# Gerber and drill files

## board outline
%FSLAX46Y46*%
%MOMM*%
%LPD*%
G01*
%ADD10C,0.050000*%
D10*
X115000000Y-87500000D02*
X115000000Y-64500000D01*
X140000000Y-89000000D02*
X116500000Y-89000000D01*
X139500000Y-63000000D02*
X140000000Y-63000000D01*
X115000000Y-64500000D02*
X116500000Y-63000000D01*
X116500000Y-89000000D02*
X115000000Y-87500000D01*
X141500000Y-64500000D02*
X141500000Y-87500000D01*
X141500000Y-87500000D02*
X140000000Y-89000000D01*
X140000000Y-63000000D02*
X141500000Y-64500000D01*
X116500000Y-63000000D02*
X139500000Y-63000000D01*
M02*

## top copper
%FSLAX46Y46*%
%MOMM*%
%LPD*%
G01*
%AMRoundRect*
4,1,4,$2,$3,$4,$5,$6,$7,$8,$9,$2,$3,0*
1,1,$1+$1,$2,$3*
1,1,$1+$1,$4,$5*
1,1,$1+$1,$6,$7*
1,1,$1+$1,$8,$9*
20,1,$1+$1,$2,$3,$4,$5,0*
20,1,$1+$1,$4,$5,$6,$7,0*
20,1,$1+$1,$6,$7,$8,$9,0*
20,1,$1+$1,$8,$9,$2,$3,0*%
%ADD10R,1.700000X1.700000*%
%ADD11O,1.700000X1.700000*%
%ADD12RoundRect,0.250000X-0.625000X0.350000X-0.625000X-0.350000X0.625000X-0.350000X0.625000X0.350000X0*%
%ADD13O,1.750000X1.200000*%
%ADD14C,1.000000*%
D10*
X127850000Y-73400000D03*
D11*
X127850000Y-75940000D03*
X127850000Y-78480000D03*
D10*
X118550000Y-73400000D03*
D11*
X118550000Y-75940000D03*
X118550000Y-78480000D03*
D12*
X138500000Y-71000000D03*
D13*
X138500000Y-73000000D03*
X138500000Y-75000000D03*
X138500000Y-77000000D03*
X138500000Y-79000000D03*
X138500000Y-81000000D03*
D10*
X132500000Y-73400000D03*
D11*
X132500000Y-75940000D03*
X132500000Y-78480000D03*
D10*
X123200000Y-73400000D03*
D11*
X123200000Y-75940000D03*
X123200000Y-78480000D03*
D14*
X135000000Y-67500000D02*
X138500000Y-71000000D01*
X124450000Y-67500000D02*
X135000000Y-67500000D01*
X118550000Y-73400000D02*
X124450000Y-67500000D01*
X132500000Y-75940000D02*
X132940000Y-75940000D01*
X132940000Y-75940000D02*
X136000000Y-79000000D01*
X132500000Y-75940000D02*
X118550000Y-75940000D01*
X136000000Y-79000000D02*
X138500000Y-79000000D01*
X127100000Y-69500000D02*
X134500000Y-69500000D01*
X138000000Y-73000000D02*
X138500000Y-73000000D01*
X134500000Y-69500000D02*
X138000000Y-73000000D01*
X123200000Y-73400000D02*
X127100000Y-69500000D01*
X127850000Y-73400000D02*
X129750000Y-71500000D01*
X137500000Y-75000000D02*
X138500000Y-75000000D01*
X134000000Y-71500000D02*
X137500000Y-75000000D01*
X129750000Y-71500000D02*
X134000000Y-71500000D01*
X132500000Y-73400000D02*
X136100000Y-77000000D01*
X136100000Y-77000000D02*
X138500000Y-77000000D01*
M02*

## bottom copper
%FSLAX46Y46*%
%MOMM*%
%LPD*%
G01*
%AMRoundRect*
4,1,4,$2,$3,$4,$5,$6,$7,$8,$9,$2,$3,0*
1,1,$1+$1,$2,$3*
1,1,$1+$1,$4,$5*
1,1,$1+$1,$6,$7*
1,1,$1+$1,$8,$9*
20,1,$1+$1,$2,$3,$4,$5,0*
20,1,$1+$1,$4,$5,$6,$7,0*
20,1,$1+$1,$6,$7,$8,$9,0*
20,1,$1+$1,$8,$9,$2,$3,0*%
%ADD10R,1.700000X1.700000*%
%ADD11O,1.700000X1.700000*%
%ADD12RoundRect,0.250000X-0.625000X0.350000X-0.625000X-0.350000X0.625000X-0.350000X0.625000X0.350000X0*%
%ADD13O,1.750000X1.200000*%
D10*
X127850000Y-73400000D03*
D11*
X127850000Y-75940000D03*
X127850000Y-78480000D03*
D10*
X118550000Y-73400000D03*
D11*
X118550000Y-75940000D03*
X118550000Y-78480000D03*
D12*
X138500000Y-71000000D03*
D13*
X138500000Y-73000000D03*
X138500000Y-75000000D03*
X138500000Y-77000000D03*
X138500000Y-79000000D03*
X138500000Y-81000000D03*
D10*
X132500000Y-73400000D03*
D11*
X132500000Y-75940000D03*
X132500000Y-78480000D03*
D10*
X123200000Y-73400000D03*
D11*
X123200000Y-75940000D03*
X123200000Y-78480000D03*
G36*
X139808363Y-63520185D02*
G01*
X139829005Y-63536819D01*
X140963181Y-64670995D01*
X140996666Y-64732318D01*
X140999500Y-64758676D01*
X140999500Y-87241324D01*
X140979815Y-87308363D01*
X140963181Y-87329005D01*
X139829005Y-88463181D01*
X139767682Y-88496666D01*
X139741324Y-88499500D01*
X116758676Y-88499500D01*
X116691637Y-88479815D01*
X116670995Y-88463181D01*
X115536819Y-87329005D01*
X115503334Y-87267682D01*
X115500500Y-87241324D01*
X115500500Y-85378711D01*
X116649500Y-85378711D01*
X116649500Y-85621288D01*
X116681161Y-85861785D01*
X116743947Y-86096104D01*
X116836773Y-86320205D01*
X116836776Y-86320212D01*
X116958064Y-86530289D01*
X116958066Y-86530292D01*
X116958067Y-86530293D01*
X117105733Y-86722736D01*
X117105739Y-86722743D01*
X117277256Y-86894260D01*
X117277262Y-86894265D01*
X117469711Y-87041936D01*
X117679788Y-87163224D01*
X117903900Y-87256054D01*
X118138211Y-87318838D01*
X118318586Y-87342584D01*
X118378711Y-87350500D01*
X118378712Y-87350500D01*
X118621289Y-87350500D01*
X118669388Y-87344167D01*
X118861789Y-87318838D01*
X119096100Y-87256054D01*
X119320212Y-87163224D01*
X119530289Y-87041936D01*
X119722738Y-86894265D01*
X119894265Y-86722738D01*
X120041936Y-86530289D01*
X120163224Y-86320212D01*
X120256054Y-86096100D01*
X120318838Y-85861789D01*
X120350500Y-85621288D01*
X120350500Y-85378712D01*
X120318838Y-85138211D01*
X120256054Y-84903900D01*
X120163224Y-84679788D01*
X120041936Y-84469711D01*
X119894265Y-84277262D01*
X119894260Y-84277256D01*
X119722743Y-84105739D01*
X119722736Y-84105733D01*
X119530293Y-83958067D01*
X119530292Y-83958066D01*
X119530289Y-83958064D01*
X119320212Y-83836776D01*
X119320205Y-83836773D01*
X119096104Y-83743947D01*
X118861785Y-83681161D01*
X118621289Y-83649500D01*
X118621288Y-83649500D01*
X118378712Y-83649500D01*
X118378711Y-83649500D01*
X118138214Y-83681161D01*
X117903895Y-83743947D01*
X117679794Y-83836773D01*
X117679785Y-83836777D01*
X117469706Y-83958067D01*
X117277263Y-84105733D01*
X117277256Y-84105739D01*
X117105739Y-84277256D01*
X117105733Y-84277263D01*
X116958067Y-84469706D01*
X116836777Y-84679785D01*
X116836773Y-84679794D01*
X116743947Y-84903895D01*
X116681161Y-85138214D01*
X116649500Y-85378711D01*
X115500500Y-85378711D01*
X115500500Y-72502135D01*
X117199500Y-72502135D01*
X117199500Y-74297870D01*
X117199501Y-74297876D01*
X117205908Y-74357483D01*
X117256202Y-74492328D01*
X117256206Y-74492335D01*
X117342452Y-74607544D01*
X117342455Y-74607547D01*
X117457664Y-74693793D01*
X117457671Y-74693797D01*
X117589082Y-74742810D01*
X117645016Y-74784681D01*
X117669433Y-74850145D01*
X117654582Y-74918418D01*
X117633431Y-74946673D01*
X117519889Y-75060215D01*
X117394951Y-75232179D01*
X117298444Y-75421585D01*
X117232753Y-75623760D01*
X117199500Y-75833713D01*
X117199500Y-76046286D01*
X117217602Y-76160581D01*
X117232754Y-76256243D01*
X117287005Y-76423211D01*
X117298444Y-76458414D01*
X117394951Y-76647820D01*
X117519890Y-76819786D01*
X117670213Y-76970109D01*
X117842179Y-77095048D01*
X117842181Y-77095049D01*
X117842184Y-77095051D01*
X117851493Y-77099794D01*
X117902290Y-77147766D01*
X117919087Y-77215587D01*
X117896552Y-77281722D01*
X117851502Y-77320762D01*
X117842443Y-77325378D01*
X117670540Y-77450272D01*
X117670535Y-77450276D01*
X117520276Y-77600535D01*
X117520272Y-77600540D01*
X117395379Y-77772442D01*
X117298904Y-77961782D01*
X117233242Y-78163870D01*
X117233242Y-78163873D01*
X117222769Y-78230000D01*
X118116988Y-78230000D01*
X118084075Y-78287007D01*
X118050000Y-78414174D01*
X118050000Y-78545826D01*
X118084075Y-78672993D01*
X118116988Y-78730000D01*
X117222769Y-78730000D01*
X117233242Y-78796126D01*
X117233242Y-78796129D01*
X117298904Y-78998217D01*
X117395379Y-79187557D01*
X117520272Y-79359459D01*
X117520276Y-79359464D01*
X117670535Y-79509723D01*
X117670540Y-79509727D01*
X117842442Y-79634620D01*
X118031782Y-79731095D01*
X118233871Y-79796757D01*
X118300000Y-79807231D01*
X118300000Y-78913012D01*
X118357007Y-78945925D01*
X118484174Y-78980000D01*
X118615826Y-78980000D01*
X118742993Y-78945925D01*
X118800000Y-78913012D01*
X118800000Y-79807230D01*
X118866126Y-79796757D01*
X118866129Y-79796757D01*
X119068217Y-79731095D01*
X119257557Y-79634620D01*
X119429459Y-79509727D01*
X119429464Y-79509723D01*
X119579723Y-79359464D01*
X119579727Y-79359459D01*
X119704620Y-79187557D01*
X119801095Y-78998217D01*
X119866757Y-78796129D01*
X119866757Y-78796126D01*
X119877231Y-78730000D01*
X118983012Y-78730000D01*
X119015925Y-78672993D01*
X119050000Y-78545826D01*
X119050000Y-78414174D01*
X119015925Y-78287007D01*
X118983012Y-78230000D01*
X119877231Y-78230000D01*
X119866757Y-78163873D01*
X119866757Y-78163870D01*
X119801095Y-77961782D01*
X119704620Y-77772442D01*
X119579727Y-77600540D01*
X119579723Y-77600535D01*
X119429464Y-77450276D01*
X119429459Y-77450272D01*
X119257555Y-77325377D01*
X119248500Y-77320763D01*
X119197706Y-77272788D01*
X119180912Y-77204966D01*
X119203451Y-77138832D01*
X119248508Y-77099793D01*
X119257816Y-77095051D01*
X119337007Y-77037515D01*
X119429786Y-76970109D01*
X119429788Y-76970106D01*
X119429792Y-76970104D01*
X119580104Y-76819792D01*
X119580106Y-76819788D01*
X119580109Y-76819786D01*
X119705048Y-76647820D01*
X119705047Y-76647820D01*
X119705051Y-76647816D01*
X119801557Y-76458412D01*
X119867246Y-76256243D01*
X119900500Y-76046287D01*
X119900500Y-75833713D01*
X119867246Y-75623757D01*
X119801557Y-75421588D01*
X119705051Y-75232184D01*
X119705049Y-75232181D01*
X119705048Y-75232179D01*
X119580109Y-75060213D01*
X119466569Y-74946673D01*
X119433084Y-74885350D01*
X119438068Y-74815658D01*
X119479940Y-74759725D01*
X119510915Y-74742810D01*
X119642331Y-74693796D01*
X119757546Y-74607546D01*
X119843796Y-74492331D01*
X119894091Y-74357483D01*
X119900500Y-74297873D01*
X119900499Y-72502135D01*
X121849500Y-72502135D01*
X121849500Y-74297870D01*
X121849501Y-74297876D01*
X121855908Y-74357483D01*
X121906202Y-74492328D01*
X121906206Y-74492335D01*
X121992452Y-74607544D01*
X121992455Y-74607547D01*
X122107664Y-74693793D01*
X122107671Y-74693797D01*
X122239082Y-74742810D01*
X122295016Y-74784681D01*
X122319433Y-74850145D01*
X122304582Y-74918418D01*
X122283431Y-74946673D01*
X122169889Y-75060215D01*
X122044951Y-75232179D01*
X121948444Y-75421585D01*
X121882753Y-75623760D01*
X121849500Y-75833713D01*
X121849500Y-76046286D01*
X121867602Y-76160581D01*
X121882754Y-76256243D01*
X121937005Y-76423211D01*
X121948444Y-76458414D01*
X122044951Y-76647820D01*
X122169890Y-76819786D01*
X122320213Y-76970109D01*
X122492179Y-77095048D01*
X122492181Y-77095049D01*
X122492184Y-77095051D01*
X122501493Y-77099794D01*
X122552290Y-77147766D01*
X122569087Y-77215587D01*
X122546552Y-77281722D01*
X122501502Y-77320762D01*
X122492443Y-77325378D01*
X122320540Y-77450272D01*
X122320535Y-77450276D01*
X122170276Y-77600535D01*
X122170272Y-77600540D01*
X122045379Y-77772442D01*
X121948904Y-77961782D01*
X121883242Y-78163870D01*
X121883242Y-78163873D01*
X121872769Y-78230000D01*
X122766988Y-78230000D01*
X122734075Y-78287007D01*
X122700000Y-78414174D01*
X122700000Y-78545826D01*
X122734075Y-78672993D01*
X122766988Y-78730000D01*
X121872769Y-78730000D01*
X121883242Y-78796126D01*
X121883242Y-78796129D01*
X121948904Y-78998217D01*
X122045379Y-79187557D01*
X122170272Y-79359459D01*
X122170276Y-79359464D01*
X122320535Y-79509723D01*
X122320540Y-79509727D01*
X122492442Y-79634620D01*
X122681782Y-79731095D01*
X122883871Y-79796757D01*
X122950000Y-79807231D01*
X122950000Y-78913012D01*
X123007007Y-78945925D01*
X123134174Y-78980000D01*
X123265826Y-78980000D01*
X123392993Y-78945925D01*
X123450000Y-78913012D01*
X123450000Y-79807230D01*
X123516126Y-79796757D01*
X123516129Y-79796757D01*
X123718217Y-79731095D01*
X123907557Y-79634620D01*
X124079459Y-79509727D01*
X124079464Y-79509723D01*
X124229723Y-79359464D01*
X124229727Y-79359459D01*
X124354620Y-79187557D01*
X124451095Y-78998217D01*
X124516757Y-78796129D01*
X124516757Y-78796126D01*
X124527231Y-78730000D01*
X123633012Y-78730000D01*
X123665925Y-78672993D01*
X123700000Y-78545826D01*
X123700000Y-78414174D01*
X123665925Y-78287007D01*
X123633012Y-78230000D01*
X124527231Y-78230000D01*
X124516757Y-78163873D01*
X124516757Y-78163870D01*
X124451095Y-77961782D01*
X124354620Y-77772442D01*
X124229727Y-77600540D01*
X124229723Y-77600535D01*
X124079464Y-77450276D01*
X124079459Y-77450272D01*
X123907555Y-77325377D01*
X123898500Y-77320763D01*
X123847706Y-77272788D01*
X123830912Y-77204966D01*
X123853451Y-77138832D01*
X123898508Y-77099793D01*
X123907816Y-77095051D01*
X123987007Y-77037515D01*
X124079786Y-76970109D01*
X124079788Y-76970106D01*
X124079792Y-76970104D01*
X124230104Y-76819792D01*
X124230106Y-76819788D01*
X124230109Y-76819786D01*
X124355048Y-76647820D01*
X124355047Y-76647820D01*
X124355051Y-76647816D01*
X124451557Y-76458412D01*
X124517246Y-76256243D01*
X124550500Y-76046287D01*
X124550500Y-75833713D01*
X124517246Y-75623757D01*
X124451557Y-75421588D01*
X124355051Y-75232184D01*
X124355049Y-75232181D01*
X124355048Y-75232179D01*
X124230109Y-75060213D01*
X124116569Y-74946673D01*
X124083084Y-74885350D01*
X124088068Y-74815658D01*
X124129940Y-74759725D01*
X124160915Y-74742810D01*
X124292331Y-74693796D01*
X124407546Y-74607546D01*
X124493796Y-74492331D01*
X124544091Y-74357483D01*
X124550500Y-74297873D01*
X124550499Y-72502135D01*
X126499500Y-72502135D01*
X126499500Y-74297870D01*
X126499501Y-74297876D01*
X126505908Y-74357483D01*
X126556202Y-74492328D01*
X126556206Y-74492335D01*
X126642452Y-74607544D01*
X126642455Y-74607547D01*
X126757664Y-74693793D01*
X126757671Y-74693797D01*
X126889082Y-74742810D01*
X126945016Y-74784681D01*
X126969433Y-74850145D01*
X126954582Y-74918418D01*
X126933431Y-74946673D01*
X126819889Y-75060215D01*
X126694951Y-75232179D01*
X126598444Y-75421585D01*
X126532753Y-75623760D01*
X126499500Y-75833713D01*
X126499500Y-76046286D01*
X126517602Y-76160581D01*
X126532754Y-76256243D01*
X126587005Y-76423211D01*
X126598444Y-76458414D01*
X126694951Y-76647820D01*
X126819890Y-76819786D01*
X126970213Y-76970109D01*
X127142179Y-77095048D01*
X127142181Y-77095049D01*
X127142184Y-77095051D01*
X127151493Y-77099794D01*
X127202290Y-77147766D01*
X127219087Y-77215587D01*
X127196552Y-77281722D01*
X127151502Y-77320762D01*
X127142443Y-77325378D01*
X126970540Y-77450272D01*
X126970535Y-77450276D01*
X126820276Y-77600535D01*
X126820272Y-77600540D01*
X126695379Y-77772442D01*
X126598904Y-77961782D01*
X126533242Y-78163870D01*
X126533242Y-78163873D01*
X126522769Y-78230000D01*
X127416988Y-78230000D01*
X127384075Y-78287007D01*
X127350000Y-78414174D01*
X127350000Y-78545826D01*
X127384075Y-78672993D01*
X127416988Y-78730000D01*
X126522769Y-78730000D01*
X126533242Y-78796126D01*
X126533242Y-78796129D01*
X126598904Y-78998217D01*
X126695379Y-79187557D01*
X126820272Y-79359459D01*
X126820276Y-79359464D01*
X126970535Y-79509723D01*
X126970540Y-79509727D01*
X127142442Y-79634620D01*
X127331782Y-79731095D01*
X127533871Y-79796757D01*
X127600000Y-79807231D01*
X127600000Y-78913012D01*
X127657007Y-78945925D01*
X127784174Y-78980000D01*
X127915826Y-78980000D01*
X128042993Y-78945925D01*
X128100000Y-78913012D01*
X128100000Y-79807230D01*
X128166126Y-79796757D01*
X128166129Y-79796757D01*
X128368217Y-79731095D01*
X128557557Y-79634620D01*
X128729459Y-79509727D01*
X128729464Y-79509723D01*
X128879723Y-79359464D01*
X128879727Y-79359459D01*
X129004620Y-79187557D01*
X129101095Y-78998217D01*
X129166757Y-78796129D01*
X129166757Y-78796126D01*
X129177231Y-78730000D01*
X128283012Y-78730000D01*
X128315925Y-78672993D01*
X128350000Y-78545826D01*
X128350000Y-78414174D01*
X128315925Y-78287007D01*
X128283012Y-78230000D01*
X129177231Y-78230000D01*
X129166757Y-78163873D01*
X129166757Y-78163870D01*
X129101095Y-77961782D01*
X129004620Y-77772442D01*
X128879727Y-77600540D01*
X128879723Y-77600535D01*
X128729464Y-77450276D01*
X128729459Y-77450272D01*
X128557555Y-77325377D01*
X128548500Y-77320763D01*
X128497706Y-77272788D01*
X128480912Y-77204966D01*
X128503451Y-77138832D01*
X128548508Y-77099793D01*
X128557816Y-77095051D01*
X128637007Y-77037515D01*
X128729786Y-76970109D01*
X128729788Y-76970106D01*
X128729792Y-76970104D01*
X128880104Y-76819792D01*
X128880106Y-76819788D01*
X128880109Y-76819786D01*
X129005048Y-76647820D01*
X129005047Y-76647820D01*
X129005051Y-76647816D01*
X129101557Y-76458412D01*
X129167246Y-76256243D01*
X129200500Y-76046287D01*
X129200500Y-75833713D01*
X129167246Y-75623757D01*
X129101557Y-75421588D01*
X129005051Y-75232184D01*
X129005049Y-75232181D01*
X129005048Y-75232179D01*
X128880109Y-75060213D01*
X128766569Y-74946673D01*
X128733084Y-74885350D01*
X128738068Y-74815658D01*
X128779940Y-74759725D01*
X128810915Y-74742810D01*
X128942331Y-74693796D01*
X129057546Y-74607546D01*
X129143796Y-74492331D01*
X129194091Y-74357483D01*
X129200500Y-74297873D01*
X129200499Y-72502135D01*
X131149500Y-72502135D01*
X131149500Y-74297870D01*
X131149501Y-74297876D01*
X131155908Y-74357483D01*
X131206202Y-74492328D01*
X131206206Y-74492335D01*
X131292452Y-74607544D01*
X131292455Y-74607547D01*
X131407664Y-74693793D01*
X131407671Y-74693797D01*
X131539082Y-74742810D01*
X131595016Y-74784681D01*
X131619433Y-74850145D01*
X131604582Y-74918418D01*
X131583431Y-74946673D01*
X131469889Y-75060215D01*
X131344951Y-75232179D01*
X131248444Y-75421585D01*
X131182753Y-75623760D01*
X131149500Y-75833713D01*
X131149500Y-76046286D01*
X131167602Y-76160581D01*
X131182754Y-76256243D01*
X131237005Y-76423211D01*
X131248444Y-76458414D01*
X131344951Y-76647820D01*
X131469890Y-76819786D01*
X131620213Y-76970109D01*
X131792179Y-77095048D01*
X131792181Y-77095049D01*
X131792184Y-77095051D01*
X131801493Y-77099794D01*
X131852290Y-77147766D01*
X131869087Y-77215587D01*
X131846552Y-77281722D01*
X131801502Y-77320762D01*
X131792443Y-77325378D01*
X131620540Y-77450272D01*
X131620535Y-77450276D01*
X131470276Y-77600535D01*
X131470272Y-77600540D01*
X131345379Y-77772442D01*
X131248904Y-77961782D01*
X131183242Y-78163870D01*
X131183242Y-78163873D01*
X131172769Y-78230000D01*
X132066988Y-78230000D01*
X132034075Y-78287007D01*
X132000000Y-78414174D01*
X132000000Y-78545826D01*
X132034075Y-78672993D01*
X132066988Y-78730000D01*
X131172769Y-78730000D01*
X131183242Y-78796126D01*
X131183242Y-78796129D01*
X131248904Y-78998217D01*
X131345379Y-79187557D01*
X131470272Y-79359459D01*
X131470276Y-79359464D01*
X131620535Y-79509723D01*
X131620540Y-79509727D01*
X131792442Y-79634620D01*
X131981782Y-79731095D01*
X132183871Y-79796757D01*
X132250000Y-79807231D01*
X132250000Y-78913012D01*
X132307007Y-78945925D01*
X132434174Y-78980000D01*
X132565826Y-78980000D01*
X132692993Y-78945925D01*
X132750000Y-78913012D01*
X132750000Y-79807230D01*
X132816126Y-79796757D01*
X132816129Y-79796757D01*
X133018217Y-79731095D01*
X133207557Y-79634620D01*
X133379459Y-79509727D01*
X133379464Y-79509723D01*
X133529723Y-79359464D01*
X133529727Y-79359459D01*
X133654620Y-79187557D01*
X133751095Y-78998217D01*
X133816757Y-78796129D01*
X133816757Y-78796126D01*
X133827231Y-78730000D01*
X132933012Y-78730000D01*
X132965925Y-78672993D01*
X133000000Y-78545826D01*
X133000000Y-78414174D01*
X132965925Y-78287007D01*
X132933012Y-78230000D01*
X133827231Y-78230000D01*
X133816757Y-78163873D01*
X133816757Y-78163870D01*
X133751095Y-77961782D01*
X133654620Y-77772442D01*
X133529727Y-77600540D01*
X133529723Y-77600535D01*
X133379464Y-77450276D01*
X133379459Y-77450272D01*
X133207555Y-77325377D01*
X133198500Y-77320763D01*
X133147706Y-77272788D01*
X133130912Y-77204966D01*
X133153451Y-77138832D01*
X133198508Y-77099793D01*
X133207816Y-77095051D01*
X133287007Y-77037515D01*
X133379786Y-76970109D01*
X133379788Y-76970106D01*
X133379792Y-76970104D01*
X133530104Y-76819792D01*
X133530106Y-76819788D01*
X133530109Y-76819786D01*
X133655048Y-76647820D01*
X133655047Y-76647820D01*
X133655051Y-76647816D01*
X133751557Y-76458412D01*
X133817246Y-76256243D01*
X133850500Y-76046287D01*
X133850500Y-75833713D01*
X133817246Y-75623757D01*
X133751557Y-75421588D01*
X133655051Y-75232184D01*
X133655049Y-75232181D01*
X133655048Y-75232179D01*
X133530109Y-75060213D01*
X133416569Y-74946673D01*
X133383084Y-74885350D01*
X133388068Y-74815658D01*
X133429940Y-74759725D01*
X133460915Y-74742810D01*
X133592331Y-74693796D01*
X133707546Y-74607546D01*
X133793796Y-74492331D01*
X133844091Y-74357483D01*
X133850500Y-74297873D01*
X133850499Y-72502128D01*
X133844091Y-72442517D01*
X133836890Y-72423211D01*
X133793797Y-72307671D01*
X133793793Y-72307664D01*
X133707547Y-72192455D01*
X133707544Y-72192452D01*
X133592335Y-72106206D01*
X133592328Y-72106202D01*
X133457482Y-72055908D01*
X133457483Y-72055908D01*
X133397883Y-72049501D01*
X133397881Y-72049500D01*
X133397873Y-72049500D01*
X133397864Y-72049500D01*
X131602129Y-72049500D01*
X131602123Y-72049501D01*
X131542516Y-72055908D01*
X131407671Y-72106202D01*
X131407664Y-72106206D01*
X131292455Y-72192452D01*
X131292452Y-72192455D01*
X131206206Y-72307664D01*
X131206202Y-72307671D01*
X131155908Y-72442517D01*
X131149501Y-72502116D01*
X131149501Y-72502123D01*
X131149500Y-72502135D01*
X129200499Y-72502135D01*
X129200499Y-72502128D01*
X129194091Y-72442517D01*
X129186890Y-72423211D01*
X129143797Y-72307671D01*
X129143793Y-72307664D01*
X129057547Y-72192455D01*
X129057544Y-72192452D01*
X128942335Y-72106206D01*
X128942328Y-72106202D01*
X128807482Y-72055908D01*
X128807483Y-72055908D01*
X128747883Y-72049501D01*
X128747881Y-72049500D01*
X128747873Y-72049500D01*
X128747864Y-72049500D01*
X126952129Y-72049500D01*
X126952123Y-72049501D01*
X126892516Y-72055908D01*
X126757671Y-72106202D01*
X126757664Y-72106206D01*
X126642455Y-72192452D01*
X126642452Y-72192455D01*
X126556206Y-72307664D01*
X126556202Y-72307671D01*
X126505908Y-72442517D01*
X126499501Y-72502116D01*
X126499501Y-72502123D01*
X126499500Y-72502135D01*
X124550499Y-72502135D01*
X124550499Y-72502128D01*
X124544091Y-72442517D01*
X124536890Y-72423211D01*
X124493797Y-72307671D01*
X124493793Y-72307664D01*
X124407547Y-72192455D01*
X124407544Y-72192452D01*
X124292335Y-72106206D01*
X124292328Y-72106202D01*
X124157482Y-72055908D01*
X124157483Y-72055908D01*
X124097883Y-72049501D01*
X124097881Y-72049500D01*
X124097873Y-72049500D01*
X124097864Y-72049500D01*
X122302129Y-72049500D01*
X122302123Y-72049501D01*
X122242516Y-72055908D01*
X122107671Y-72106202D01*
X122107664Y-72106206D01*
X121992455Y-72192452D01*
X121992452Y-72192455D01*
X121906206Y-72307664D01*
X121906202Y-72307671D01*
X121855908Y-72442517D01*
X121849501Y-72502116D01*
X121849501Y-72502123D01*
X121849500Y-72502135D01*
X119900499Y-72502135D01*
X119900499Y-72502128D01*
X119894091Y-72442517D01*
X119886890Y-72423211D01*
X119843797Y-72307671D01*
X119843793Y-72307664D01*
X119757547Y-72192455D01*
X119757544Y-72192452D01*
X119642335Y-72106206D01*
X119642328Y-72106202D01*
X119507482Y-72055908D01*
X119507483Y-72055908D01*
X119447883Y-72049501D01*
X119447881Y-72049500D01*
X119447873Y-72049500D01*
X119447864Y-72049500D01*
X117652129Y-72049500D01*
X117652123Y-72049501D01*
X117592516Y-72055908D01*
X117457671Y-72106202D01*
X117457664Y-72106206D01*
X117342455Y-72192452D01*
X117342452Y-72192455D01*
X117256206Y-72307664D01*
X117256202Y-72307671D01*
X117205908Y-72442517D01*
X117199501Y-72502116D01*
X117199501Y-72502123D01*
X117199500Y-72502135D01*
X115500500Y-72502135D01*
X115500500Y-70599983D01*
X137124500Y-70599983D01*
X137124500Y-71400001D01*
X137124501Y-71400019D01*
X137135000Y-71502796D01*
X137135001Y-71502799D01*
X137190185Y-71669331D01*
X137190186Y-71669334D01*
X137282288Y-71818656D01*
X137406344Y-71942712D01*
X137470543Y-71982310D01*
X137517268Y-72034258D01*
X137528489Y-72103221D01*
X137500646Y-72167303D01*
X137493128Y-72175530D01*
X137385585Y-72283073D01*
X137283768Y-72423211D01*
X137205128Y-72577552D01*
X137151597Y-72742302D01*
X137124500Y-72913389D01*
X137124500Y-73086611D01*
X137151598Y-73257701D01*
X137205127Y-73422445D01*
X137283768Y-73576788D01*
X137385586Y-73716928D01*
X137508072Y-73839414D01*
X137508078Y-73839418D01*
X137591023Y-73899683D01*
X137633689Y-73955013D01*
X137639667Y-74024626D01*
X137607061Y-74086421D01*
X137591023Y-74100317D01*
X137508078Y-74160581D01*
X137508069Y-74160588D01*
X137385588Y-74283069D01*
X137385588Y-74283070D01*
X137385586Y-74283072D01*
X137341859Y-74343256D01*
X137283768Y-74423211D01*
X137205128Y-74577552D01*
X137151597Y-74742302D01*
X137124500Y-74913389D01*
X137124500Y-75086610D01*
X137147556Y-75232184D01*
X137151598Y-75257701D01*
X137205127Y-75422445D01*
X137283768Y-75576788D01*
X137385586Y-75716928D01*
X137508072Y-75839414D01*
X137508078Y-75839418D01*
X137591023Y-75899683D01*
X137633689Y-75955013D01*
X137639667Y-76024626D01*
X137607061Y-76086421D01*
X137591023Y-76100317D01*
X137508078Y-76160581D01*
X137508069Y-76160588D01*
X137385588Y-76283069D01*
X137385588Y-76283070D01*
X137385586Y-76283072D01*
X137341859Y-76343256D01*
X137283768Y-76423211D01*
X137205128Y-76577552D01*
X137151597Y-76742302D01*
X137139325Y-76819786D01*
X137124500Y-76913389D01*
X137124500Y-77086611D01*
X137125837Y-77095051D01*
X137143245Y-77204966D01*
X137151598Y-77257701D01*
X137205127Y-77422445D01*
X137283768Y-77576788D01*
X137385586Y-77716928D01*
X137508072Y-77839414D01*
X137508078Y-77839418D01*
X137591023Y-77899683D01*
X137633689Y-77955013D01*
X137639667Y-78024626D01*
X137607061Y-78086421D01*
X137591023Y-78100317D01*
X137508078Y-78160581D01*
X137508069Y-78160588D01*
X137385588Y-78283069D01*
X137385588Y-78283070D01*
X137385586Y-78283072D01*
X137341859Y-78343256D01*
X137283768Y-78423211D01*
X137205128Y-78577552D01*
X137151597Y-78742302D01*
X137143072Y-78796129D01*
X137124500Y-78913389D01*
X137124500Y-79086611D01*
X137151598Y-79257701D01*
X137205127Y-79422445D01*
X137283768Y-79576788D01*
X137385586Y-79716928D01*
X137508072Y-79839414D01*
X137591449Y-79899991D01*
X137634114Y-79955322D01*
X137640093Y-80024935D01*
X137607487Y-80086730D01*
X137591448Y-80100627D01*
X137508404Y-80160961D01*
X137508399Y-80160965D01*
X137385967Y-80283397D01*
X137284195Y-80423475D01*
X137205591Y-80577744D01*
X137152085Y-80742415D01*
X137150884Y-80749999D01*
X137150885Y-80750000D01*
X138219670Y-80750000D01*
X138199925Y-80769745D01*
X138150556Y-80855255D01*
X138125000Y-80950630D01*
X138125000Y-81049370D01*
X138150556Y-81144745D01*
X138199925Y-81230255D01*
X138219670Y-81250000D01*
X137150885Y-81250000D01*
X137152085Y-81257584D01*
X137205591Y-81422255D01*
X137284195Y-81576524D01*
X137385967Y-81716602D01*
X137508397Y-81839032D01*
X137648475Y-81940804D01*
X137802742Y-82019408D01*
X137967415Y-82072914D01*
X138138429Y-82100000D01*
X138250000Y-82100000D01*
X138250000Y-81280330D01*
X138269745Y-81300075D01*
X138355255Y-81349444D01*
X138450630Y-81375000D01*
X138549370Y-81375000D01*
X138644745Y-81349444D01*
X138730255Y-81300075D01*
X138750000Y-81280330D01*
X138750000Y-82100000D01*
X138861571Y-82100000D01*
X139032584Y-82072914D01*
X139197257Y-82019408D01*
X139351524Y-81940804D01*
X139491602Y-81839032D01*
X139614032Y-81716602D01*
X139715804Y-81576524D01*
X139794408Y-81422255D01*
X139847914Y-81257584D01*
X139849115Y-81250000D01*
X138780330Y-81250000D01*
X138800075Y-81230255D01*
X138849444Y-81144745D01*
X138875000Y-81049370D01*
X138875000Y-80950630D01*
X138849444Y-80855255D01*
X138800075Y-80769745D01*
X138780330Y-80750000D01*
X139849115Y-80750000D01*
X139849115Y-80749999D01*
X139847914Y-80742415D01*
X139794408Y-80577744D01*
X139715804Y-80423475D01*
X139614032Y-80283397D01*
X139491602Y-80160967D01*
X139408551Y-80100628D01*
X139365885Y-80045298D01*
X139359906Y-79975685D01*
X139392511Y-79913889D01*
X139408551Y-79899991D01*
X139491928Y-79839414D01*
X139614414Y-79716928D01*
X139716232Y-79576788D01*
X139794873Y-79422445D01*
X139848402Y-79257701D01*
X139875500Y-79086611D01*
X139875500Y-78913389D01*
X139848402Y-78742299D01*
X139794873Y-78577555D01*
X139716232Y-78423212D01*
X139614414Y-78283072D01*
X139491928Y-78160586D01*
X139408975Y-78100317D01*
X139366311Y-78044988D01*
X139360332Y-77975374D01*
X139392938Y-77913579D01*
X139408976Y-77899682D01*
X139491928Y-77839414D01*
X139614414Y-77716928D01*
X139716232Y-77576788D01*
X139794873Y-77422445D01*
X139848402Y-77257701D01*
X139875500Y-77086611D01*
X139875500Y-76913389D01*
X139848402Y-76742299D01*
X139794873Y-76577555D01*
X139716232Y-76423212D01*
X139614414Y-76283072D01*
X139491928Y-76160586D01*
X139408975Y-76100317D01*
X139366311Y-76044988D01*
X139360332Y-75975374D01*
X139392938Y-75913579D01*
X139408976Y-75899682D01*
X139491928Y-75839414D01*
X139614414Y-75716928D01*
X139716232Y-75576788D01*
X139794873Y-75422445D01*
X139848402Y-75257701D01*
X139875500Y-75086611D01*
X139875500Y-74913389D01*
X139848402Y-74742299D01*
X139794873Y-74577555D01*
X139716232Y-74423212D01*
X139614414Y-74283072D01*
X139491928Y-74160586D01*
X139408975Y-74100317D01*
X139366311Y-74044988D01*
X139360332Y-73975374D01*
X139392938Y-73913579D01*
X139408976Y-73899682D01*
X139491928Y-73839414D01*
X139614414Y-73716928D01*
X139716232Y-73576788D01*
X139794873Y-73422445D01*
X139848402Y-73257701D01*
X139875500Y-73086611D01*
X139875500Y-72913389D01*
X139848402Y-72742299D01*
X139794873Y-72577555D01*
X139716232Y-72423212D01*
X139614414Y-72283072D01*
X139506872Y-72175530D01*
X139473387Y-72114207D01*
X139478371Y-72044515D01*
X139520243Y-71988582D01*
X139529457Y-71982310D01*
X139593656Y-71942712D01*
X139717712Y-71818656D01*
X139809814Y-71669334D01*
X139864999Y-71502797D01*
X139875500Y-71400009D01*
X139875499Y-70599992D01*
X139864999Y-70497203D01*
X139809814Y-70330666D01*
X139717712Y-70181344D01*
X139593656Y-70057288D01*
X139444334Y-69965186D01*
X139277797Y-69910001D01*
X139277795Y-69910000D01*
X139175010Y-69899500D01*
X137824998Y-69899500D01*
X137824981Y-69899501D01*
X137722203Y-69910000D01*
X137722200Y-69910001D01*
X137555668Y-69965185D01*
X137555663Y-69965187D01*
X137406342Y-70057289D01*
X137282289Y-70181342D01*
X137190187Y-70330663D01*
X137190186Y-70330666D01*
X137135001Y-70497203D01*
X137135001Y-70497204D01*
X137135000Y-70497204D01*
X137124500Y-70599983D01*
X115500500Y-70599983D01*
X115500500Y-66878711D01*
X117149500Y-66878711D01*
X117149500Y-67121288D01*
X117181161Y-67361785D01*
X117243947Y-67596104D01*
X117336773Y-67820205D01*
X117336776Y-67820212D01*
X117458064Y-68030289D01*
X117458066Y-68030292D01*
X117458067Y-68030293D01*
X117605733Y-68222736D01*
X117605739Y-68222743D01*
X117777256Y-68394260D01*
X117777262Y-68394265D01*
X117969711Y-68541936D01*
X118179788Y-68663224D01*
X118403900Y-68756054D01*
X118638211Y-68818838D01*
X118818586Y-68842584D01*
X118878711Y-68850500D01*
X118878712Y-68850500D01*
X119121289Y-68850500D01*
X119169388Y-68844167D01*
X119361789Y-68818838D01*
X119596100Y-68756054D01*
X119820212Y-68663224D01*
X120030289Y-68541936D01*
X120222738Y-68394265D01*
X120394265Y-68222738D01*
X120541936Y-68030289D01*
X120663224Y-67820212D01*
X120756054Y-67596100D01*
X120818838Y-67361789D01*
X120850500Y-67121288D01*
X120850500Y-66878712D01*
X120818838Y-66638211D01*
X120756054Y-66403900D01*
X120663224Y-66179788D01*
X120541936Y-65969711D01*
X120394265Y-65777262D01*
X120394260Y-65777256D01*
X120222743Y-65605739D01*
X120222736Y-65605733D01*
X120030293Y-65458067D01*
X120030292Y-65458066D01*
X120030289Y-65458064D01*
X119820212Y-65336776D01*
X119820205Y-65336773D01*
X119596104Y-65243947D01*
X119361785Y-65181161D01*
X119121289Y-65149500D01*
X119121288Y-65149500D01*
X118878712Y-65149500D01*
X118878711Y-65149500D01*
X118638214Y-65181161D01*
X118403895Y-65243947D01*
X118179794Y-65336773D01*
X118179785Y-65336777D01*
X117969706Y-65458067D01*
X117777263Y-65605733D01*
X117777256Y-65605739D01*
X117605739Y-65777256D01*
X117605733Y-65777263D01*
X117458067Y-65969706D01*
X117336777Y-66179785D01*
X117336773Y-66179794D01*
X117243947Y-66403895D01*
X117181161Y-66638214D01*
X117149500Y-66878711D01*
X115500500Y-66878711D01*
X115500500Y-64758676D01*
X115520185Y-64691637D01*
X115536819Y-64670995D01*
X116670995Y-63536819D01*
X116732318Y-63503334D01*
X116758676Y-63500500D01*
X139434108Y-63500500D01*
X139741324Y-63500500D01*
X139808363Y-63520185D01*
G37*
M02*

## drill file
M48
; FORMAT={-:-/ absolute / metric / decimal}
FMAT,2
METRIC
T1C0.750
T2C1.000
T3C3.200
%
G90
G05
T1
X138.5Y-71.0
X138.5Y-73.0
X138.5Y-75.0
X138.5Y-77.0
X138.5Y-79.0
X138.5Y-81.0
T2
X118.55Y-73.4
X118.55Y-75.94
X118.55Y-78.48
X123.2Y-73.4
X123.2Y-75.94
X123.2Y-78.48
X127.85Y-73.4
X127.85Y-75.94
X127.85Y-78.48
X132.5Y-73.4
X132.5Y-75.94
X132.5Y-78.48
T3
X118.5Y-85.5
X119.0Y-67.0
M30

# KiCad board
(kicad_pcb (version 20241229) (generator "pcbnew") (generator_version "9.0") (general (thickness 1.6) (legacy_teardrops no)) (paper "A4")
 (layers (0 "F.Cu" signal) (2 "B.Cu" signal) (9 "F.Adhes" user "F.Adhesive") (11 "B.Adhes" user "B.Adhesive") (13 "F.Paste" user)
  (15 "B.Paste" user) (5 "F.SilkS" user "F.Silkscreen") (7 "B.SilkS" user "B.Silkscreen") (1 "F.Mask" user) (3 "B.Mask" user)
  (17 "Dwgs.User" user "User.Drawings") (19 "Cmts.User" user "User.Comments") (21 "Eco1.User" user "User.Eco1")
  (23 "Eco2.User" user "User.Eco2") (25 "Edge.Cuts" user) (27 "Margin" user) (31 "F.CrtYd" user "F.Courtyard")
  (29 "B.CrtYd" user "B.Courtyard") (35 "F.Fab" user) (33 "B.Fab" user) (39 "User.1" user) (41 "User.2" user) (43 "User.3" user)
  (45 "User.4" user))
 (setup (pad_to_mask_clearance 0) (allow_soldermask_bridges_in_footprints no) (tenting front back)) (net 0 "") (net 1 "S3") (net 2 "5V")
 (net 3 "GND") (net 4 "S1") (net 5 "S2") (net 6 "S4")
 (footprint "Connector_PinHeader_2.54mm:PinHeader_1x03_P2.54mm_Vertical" (layer "F.Cu") (at 127.85 73.4)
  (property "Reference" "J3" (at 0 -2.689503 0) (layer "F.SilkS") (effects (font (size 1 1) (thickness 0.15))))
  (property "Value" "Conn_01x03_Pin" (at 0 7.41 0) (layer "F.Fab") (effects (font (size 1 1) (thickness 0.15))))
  (pad "1" thru_hole rect (at 0 0) (size 1.7 1.7) (drill 1) (layers "*.Cu" "*.Mask") (remove_unused_layers no) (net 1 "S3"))
  (pad "2" thru_hole oval (at 0 2.54) (size 1.7 1.7) (drill 1) (layers "*.Cu" "*.Mask") (remove_unused_layers no) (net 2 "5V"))
  (pad "3" thru_hole oval (at 0 5.08) (size 1.7 1.7) (drill 1) (layers "*.Cu" "*.Mask") (remove_unused_layers no) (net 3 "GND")))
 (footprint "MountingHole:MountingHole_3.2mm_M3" (layer "F.Cu") (at 118.5 85.5)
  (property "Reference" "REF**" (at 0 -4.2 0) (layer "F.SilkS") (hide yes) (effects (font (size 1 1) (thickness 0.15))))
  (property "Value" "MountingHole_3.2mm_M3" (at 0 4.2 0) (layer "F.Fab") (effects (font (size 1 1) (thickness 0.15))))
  (pad "" np_thru_hole circle (at 0 0) (size 3.2 3.2) (drill 3.2) (layers "*.Cu" "*.Mask")))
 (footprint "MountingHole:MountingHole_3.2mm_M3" (layer "F.Cu") (at 119 67)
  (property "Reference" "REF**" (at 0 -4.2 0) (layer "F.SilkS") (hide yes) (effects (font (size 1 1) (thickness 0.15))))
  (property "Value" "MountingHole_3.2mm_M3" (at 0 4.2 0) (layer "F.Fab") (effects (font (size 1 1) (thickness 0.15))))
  (pad "" np_thru_hole circle (at 0 0) (size 3.2 3.2) (drill 3.2) (layers "*.Cu" "*.Mask")))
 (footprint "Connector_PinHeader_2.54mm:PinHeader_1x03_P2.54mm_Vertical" (layer "F.Cu") (at 118.55 73.4)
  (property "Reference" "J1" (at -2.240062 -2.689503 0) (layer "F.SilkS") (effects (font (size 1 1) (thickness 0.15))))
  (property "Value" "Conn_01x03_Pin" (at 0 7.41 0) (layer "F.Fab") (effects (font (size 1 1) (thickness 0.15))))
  (pad "1" thru_hole rect (at 0 0) (size 1.7 1.7) (drill 1) (layers "*.Cu" "*.Mask") (remove_unused_layers no) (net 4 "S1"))
  (pad "2" thru_hole oval (at 0 2.54) (size 1.7 1.7) (drill 1) (layers "*.Cu" "*.Mask") (remove_unused_layers no) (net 2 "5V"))
  (pad "3" thru_hole oval (at 0 5.08) (size 1.7 1.7) (drill 1) (layers "*.Cu" "*.Mask") (remove_unused_layers no) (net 3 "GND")))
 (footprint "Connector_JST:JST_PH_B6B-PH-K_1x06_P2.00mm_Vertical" (layer "F.Cu") (at 138.5 71 -90)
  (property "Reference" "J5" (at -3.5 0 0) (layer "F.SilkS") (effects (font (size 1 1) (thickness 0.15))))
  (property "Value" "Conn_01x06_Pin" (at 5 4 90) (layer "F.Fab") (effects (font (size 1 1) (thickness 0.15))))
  (pad "1" thru_hole roundrect (at 0 0 270) (size 1.2 1.75) (drill 0.75) (layers "*.Cu" "*.Mask") (remove_unused_layers no)
   (roundrect_rratio 0.208333) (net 4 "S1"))
  (pad "2" thru_hole oval (at 2 0 270) (size 1.2 1.75) (drill 0.75) (layers "*.Cu" "*.Mask") (remove_unused_layers no) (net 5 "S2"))
  (pad "3" thru_hole oval (at 4 0 270) (size 1.2 1.75) (drill 0.75) (layers "*.Cu" "*.Mask") (remove_unused_layers no) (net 1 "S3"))
  (pad "4" thru_hole oval (at 6 0 270) (size 1.2 1.75) (drill 0.75) (layers "*.Cu" "*.Mask") (remove_unused_layers no) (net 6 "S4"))
  (pad "5" thru_hole oval (at 8 0 270) (size 1.2 1.75) (drill 0.75) (layers "*.Cu" "*.Mask") (remove_unused_layers no) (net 2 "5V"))
  (pad "6" thru_hole oval (at 10 0 270) (size 1.2 1.75) (drill 0.75) (layers "*.Cu" "*.Mask") (remove_unused_layers no) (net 3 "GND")))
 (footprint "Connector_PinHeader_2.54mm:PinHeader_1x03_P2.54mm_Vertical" (layer "F.Cu") (at 132.5 73.4)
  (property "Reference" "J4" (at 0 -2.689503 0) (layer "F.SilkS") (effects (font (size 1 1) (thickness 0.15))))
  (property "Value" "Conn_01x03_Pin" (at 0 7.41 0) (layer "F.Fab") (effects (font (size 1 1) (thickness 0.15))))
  (pad "1" thru_hole rect (at 0 0) (size 1.7 1.7) (drill 1) (layers "*.Cu" "*.Mask") (remove_unused_layers no) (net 6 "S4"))
  (pad "2" thru_hole oval (at 0 2.54) (size 1.7 1.7) (drill 1) (layers "*.Cu" "*.Mask") (remove_unused_layers no) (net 2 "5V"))
  (pad "3" thru_hole oval (at 0 5.08) (size 1.7 1.7) (drill 1) (layers "*.Cu" "*.Mask") (remove_unused_layers no) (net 3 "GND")))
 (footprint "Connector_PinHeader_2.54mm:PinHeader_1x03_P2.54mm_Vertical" (layer "F.Cu") (at 123.2 73.4)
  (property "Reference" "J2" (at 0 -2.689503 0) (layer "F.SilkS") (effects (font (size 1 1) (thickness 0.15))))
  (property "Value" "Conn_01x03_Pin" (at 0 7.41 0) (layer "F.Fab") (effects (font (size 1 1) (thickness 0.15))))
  (pad "1" thru_hole rect (at 0 0) (size 1.7 1.7) (drill 1) (layers "*.Cu" "*.Mask") (remove_unused_layers no) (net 5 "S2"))
  (pad "2" thru_hole oval (at 0 2.54) (size 1.7 1.7) (drill 1) (layers "*.Cu" "*.Mask") (remove_unused_layers no) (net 2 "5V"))
  (pad "3" thru_hole oval (at 0 5.08) (size 1.7 1.7) (drill 1) (layers "*.Cu" "*.Mask") (remove_unused_layers no) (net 3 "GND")))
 (gr_line (start 115 87.5) (end 115 64.5) (stroke (width 0.05) (type default)) (layer "Edge.Cuts"))
 (gr_line (start 140 89) (end 116.5 89) (stroke (width 0.05) (type default)) (layer "Edge.Cuts"))
 (gr_line (start 139.5 63) (end 140 63) (stroke (width 0.05) (type default)) (layer "Edge.Cuts"))
 (gr_line (start 115 64.5) (end 116.5 63) (stroke (width 0.05) (type default)) (layer "Edge.Cuts"))
 (gr_line (start 116.5 89) (end 115 87.5) (stroke (width 0.05) (type default)) (layer "Edge.Cuts"))
 (gr_line (start 141.5 64.5) (end 141.5 87.5) (stroke (width 0.05) (type default)) (layer "Edge.Cuts"))
 (gr_line (start 141.5 87.5) (end 140 89) (stroke (width 0.05) (type default)) (layer "Edge.Cuts"))
 (gr_line (start 140 63) (end 141.5 64.5) (stroke (width 0.05) (type default)) (layer "Edge.Cuts"))
 (gr_line (start 116.5 63) (end 139.5 63) (stroke (width 0.05) (type default)) (layer "Edge.Cuts"))
 (segment (start 135 67.5) (end 138.5 71) (width 1) (layer "F.Cu") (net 4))
 (segment (start 124.45 67.5) (end 135 67.5) (width 1) (layer "F.Cu") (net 4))
 (segment (start 118.55 73.4) (end 124.45 67.5) (width 1) (layer "F.Cu") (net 4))
 (segment (start 132.5 75.94) (end 132.94 75.94) (width 1) (layer "F.Cu") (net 2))
 (segment (start 132.94 75.94) (end 136 79) (width 1) (layer "F.Cu") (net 2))
 (segment (start 132.5 75.94) (end 118.55 75.94) (width 1) (layer "F.Cu") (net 2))
 (segment (start 136 79) (end 138.5 79) (width 1) (layer "F.Cu") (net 2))
 (segment (start 127.1 69.5) (end 134.5 69.5) (width 1) (layer "F.Cu") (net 5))
 (segment (start 138 73) (end 138.5 73) (width 1) (layer "F.Cu") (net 5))
 (segment (start 134.5 69.5) (end 138 73) (width 1) (layer "F.Cu") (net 5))
 (segment (start 123.2 73.4) (end 127.1 69.5) (width 1) (layer "F.Cu") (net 5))
 (segment (start 127.85 73.4) (end 129.75 71.5) (width 1) (layer "F.Cu") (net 1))
 (segment (start 137.5 75) (end 138.5 75) (width 1) (layer "F.Cu") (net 1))
 (segment (start 134 71.5) (end 137.5 75) (width 1) (layer "F.Cu") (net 1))
 (segment (start 129.75 71.5) (end 134 71.5) (width 1) (layer "F.Cu") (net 1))
 (segment (start 132.5 73.4) (end 136.1 77) (width 1) (layer "F.Cu") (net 6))
 (segment (start 136.1 77) (end 138.5 77) (width 1) (layer "F.Cu") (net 6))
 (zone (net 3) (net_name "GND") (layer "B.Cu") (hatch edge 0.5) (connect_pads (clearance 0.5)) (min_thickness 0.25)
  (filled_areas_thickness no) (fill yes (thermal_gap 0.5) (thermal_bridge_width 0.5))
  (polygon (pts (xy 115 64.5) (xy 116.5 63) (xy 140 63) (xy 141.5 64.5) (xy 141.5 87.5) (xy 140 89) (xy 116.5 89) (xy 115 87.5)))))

